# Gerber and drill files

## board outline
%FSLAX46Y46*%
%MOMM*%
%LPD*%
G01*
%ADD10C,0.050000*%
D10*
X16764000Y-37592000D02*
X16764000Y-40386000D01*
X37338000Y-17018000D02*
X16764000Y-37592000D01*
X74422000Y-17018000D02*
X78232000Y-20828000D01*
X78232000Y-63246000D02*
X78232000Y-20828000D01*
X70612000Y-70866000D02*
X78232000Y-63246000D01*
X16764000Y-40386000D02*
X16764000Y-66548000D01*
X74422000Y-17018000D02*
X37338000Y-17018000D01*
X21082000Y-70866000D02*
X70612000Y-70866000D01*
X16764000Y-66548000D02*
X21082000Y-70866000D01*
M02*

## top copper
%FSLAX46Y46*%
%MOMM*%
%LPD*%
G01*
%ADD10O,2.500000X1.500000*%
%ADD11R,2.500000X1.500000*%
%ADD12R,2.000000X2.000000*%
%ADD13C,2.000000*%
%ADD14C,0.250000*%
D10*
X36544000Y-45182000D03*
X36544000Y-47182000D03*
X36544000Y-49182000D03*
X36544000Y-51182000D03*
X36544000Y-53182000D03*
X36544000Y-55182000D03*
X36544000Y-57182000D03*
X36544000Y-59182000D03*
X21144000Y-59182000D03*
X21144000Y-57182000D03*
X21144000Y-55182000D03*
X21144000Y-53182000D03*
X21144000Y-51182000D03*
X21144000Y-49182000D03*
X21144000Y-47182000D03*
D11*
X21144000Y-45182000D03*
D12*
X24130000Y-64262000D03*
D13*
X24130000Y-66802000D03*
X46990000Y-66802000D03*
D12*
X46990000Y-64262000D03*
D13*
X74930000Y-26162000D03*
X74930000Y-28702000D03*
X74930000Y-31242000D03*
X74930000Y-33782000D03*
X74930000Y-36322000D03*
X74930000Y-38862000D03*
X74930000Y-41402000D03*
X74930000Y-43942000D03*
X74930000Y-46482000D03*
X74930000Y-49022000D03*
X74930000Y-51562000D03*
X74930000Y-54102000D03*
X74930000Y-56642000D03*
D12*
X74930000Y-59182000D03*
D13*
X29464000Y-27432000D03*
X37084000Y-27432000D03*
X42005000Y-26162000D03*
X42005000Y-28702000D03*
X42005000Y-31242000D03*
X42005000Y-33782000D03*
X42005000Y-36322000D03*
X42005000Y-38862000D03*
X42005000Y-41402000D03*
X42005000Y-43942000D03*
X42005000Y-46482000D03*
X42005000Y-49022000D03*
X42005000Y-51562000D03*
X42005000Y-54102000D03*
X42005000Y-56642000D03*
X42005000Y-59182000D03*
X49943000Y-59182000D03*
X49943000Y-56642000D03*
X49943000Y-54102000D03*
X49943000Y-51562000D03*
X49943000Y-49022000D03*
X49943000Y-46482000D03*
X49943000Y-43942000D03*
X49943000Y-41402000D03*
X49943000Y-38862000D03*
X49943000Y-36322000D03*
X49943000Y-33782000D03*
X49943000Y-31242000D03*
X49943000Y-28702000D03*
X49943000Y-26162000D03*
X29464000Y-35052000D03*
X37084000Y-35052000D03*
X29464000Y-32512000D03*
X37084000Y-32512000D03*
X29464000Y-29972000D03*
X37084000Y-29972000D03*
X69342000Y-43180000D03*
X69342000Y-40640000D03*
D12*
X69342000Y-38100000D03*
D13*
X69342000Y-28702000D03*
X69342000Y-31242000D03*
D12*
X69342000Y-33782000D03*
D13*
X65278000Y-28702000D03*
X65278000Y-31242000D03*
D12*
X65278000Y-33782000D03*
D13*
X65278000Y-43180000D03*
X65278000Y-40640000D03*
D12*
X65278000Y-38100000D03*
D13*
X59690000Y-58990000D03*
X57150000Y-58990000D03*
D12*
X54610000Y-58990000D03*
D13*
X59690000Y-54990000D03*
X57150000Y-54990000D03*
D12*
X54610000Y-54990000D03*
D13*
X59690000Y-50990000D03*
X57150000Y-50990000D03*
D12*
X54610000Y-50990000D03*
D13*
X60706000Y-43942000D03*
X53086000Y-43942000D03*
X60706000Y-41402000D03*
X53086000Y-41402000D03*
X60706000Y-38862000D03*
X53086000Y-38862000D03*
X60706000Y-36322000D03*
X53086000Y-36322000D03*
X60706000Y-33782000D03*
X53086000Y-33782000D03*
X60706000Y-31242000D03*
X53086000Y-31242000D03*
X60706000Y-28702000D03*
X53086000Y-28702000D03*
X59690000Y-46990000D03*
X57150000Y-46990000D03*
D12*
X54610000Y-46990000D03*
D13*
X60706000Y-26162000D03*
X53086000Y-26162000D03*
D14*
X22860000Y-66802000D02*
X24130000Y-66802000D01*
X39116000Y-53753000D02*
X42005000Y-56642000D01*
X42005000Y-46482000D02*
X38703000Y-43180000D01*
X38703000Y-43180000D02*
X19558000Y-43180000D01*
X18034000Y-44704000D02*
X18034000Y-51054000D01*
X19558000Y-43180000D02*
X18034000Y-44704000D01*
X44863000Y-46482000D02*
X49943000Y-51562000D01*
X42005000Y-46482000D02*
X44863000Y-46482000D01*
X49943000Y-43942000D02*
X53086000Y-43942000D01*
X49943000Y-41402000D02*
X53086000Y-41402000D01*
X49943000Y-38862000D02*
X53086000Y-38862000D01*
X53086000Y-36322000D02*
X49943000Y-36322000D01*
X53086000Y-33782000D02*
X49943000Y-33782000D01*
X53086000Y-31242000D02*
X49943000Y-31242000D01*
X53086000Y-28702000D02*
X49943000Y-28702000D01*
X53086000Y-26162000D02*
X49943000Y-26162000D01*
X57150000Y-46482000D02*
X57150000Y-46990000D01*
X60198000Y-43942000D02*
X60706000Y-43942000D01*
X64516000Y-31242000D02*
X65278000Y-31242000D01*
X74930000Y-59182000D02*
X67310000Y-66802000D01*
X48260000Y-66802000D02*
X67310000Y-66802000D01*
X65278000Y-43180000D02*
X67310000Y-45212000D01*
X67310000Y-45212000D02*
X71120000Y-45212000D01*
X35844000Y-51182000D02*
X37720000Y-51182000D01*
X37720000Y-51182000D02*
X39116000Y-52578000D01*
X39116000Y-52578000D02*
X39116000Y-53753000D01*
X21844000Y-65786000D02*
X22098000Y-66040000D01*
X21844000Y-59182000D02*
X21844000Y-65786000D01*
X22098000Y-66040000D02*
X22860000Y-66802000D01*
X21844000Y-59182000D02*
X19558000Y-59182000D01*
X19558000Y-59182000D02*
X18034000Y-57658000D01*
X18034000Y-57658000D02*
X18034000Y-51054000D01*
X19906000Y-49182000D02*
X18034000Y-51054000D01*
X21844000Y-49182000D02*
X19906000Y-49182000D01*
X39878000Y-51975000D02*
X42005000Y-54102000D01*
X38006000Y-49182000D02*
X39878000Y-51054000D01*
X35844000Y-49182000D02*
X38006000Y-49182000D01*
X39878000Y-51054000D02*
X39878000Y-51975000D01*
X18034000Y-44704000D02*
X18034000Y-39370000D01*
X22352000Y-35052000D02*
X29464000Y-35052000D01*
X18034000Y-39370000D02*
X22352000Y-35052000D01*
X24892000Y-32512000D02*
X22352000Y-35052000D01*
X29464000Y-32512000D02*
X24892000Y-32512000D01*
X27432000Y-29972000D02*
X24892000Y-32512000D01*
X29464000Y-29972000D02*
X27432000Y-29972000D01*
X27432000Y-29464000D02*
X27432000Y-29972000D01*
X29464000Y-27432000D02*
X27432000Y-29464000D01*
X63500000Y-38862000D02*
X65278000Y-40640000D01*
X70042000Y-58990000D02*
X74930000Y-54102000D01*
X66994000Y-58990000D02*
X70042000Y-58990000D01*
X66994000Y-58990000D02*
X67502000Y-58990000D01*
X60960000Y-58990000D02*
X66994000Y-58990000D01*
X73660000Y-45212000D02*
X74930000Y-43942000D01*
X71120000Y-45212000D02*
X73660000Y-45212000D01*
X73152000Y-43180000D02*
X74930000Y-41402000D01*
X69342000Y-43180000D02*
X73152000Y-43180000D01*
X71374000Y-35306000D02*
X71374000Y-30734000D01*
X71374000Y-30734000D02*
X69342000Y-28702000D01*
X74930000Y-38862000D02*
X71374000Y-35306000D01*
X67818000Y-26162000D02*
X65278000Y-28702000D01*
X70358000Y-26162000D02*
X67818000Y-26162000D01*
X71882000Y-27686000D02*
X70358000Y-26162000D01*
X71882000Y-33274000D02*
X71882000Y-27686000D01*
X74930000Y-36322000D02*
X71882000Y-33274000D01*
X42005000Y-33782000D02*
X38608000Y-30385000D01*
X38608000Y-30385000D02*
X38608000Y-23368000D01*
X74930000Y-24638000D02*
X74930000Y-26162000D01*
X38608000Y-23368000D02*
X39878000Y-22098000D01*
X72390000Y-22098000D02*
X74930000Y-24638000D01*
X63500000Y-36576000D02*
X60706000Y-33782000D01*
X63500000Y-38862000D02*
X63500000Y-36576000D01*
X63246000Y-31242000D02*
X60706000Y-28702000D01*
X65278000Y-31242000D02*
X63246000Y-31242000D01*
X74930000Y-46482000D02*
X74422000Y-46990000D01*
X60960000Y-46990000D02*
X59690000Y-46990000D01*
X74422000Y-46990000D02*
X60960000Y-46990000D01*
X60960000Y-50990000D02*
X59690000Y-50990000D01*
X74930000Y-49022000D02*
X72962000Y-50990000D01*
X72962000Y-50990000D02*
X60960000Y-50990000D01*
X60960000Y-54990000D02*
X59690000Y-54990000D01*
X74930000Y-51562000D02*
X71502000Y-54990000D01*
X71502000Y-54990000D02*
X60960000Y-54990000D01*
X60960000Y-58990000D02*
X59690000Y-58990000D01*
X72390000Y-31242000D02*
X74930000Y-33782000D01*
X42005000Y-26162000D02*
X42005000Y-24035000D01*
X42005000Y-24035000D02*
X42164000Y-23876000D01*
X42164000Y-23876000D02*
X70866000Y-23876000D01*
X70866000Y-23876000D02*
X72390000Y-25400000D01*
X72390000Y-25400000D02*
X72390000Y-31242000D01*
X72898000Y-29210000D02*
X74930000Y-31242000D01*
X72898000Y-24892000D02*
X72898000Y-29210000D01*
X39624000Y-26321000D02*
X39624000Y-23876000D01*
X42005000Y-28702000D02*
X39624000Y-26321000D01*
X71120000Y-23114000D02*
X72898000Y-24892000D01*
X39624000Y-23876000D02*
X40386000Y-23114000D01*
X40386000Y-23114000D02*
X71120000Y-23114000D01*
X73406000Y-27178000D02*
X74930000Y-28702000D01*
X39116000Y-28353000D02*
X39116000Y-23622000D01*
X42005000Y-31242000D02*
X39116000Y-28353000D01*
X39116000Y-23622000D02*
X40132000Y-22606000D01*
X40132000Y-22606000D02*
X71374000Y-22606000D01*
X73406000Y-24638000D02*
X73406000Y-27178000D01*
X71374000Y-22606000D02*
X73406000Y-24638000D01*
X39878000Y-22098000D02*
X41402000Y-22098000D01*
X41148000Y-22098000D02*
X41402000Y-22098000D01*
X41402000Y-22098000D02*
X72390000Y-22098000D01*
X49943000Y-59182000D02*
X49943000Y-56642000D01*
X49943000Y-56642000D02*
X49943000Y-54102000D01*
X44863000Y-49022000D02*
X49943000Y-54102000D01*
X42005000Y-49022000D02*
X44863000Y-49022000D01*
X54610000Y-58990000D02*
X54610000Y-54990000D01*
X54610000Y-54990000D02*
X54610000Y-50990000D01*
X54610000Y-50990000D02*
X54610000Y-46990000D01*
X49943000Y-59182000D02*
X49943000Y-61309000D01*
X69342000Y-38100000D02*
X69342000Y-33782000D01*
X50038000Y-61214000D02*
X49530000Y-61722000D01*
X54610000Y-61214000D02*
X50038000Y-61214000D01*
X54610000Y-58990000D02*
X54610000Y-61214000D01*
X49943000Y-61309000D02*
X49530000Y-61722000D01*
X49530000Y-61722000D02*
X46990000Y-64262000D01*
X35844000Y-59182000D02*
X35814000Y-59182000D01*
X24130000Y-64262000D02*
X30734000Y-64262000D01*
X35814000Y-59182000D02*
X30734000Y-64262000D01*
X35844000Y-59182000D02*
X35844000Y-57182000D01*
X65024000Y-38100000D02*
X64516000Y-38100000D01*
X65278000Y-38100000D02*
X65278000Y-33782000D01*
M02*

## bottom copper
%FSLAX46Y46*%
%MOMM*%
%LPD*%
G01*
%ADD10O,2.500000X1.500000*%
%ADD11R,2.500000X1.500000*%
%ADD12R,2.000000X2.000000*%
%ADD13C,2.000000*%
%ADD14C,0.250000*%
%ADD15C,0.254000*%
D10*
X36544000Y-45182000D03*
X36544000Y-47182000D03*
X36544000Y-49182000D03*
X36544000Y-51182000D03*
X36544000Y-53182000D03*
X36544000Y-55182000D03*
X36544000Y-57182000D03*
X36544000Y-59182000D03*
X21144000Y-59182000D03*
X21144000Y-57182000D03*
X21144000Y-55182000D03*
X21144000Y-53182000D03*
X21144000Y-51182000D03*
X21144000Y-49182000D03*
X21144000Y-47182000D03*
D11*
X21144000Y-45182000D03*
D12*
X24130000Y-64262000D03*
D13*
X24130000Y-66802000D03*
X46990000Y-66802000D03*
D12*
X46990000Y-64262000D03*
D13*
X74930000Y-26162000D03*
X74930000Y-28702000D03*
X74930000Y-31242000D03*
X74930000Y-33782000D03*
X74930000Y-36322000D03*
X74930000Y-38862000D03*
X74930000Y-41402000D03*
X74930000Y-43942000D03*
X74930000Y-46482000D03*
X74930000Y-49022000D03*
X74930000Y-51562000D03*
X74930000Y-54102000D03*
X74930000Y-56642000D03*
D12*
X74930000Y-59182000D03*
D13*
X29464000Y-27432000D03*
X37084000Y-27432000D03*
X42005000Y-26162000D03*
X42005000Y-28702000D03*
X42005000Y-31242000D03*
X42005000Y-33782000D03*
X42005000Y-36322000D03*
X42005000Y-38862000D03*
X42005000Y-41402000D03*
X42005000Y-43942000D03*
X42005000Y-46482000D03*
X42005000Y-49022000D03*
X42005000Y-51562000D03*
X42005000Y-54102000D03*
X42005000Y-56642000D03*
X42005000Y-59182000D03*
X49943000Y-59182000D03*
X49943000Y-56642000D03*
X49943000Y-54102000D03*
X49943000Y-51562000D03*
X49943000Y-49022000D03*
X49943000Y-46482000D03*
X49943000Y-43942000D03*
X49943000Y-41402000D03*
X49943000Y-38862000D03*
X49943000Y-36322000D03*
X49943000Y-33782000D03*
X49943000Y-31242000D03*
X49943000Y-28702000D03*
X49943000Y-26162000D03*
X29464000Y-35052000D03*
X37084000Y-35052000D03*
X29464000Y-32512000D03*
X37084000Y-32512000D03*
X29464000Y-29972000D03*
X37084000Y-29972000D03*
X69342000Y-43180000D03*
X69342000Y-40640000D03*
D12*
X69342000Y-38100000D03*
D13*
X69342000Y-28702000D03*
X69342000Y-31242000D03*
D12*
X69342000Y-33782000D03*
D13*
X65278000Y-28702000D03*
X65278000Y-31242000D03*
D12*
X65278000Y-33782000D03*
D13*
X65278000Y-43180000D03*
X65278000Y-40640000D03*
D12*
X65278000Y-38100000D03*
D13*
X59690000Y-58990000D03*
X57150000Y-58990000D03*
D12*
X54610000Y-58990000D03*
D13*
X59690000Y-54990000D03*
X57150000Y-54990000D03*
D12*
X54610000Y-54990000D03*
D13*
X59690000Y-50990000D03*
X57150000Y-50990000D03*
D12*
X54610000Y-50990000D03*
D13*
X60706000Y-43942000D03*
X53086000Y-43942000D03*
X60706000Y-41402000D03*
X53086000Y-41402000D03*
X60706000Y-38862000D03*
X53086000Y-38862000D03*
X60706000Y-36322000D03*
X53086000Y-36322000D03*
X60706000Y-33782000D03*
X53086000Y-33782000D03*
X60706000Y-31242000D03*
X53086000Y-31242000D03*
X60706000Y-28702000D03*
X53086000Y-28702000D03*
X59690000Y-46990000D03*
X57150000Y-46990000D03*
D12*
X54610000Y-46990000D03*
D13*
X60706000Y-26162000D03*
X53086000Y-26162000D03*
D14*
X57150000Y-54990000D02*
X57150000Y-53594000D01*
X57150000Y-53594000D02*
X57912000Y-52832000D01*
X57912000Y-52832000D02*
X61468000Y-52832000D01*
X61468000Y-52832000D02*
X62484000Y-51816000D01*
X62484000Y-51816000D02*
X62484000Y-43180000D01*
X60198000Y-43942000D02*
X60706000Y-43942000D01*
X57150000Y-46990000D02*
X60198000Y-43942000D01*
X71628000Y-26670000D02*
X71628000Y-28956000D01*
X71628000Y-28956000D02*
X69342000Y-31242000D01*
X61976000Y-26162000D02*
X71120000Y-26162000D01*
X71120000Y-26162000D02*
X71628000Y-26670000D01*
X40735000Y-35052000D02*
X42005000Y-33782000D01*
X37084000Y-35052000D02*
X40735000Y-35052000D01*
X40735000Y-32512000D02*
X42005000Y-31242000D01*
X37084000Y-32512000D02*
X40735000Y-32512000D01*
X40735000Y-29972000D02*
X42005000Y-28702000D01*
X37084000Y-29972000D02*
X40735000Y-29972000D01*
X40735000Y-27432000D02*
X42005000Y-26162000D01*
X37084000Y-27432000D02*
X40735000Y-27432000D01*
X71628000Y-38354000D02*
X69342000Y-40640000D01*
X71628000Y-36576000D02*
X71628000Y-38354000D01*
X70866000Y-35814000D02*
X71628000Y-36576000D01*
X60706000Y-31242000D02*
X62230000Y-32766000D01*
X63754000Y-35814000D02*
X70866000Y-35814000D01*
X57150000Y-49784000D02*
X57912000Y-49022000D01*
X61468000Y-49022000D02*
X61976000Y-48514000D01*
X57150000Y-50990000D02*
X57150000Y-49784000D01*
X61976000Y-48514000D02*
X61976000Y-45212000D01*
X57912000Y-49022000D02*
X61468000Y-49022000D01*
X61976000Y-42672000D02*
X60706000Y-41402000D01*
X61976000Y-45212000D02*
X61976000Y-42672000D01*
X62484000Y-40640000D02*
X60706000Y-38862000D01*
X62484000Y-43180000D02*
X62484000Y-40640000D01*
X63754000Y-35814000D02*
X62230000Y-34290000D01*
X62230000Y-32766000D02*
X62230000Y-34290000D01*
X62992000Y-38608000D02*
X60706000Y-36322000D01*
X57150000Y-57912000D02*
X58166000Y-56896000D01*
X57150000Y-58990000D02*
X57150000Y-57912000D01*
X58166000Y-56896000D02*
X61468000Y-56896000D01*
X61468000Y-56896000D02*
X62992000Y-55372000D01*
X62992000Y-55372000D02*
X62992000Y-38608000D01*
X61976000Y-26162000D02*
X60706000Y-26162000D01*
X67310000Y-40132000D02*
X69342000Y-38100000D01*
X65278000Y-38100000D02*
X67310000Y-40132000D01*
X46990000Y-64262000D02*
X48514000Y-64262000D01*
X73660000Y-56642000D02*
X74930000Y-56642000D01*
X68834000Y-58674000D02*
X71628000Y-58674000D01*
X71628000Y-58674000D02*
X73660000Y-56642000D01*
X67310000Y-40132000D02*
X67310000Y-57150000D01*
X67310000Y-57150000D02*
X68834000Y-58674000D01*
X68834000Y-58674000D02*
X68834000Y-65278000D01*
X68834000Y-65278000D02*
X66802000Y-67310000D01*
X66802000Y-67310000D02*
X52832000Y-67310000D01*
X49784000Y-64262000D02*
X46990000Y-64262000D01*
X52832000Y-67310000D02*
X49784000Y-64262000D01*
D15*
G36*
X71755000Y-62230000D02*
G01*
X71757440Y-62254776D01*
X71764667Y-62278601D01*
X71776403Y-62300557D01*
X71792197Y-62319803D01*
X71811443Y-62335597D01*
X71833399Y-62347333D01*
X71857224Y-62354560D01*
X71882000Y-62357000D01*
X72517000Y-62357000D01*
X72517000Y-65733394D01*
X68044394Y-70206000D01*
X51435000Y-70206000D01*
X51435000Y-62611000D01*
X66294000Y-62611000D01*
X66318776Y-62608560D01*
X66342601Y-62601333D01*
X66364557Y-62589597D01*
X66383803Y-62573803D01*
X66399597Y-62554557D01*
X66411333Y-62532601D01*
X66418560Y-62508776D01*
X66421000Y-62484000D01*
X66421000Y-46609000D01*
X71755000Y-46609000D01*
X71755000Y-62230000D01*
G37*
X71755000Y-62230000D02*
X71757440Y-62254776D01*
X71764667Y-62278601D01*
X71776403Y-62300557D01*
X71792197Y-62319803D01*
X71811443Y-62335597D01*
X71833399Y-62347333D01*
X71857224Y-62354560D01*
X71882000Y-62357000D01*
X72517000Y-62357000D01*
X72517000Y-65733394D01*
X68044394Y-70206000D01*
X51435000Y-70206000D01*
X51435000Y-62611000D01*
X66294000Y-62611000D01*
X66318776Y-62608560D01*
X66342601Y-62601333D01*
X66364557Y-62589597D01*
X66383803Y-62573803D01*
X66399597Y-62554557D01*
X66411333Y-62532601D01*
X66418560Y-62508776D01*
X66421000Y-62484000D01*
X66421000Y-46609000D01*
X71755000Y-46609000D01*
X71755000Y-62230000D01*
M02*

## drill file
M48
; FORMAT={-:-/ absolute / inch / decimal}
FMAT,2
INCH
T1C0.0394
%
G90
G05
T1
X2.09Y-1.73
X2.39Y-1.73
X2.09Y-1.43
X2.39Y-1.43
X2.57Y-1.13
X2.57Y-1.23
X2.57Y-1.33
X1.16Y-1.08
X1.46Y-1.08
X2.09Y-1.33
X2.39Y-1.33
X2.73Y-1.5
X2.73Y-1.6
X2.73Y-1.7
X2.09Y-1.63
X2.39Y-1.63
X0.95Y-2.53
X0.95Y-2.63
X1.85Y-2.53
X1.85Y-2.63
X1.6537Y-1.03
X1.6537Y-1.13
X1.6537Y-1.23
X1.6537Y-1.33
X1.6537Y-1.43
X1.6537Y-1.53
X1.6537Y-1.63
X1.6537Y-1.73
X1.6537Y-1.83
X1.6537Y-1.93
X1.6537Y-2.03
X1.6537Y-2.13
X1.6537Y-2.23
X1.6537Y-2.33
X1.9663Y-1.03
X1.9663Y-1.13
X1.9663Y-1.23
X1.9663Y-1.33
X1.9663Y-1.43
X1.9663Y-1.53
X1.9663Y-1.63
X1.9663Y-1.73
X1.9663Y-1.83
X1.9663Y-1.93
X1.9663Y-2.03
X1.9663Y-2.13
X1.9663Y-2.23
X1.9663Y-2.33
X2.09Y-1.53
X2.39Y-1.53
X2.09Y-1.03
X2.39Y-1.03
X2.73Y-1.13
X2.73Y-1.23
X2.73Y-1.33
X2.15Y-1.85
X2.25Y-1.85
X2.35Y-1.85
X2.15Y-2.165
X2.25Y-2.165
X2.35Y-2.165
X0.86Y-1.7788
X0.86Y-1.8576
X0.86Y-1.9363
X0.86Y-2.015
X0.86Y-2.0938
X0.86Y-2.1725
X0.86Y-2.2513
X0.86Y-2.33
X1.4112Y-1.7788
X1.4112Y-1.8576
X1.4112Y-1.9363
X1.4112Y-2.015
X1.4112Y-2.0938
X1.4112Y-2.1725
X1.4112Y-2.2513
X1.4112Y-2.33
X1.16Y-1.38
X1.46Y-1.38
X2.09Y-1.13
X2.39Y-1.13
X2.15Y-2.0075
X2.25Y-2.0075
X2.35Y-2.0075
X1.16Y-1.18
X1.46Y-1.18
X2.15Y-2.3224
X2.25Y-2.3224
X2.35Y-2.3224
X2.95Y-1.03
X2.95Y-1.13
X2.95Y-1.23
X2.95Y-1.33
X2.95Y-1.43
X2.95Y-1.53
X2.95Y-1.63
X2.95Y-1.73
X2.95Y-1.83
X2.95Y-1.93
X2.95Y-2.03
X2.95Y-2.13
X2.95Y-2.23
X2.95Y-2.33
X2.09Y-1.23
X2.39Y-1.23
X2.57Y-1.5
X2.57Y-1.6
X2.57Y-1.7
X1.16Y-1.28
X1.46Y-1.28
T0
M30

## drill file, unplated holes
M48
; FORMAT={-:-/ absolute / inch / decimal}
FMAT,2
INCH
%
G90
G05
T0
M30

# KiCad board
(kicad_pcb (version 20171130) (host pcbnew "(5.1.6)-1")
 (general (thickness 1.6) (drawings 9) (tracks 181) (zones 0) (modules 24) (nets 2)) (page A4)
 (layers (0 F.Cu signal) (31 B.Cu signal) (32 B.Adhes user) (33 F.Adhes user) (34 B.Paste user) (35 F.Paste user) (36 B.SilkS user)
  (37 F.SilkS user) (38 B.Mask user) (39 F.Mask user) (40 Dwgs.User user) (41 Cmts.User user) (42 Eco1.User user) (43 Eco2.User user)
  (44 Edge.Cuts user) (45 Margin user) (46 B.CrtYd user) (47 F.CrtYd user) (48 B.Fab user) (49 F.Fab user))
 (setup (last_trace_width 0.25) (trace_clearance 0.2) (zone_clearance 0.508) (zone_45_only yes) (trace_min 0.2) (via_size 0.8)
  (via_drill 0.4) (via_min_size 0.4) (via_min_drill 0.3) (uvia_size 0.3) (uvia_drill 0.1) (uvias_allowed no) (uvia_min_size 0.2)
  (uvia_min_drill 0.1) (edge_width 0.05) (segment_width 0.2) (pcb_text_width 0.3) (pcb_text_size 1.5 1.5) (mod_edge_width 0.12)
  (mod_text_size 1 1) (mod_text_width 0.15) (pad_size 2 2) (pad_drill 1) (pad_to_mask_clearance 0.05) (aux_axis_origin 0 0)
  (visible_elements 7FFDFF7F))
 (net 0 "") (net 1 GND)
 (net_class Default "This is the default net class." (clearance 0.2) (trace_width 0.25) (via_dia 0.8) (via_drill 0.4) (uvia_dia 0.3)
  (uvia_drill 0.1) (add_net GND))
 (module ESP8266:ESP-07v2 (layer F.Cu) (at 21.844 45.182)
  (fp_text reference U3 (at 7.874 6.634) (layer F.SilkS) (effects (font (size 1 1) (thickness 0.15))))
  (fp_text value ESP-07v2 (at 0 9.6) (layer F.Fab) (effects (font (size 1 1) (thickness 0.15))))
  (pad 16 thru_hole oval (at 14 0) (size 2.5 1.5) (drill 1 (offset 0.7 0)) (layers *.Cu *.Mask F.Paste F.SilkS))
  (pad 15 thru_hole oval (at 14 2) (size 2.5 1.5) (drill 1 (offset 0.7 0)) (layers *.Cu *.Mask F.Paste F.SilkS))
  (pad 14 thru_hole oval (at 14 4) (size 2.5 1.5) (drill 1 (offset 0.7 0)) (layers *.Cu *.Mask F.Paste F.SilkS))
  (pad 13 thru_hole oval (at 14 6) (size 2.5 1.5) (drill 1 (offset 0.7 0)) (layers *.Cu *.Mask F.Paste F.SilkS))
  (pad 12 thru_hole oval (at 14 8) (size 2.5 1.5) (drill 1 (offset 0.7 0)) (layers *.Cu *.Mask F.Paste F.SilkS))
  (pad 11 thru_hole oval (at 14 10) (size 2.5 1.5) (drill 1 (offset 0.7 0)) (layers *.Cu *.Mask F.Paste F.SilkS))
  (pad 10 thru_hole oval (at 14 12) (size 2.5 1.5) (drill 1 (offset 0.7 0)) (layers *.Cu *.Mask F.Paste F.SilkS) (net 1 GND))
  (pad 9 thru_hole oval (at 14 14) (size 2.5 1.5) (drill 1 (offset 0.7 0)) (layers *.Cu *.Mask F.Paste F.SilkS) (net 1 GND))
  (pad 8 thru_hole oval (at 0 14) (size 2.5 1.5) (drill 1 (offset -0.7 0)) (layers *.Cu *.Mask F.Paste F.SilkS))
  (pad 7 thru_hole oval (at 0 12) (size 2.5 1.5) (drill 1 (offset -0.7 0)) (layers *.Cu *.Mask F.Paste F.SilkS))
  (pad 6 thru_hole oval (at 0 10) (size 2.5 1.5) (drill 1 (offset -0.7 0)) (layers *.Cu *.Mask F.Paste F.SilkS))
  (pad 5 thru_hole oval (at 0 8) (size 2.5 1.5) (drill 1 (offset -0.7 0)) (layers *.Cu *.Mask F.Paste F.SilkS))
  (pad 4 thru_hole oval (at 0 6) (size 2.5 1.5) (drill 1 (offset -0.7 0)) (layers *.Cu *.Mask F.Paste F.SilkS))
  (pad 3 thru_hole oval (at 0 4) (size 2.5 1.5) (drill 1 (offset -0.7 0)) (layers *.Cu *.Mask F.Paste F.SilkS))
  (pad 2 thru_hole oval (at 0 2) (size 2.5 1.5) (drill 1 (offset -0.7 0)) (layers *.Cu *.Mask F.Paste F.SilkS))
  (pad 1 thru_hole rect (at 0 0) (size 2.5 1.5) (drill 1 (offset -0.7 0)) (layers *.Cu *.Mask F.Paste F.SilkS)))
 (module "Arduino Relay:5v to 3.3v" (layer F.Cu) (at 35.56 65.532 270)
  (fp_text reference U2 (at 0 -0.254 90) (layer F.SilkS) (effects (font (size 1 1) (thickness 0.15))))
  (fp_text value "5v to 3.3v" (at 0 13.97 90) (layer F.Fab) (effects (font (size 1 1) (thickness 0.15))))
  (pad 1 thru_hole rect (at -1.27 11.43 270) (size 2 2) (drill 1) (layers *.Cu *.Mask) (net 1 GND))
  (pad 3 thru_hole circle (at 1.27 11.43 270) (size 2 2) (drill 1) (layers *.Cu *.Mask))
  (pad 2 thru_hole circle (at 1.27 -11.43 270) (size 2 2) (drill 1) (layers *.Cu *.Mask))
  (pad 1 thru_hole rect (at -1.27 -11.43 270) (size 2 2) (drill 1) (layers *.Cu *.Mask) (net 1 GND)))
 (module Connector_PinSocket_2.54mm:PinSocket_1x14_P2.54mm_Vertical (layer F.Cu) (at 74.93 59.182 180)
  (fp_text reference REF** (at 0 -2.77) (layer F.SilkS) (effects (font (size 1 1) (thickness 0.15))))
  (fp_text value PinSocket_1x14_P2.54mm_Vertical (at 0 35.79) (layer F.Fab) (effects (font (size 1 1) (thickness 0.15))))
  (pad 14 thru_hole circle (at 0 33.02 180) (size 2 2) (drill 1) (layers *.Cu *.Mask))
  (pad 13 thru_hole circle (at 0 30.48 180) (size 2 2) (drill 1) (layers *.Cu *.Mask))
  (pad 12 thru_hole circle (at 0 27.94 180) (size 2 2) (drill 1) (layers *.Cu *.Mask))
  (pad 11 thru_hole circle (at 0 25.4 180) (size 2 2) (drill 1) (layers *.Cu *.Mask))
  (pad 10 thru_hole circle (at 0 22.86 180) (size 2 2) (drill 1) (layers *.Cu *.Mask))
  (pad 9 thru_hole circle (at 0 20.32 180) (size 2 2) (drill 1) (layers *.Cu *.Mask))
  (pad 8 thru_hole circle (at 0 17.78 180) (size 2 2) (drill 1) (layers *.Cu *.Mask))
  (pad 7 thru_hole circle (at 0 15.24 180) (size 2 2) (drill 1) (layers *.Cu *.Mask))
  (pad 6 thru_hole circle (at 0 12.7 180) (size 2 2) (drill 1) (layers *.Cu *.Mask))
  (pad 5 thru_hole circle (at 0 10.16 180) (size 2 2) (drill 1) (layers *.Cu *.Mask))
  (pad 4 thru_hole circle (at 0 7.62 180) (size 2 2) (drill 1) (layers *.Cu *.Mask))
  (pad 3 thru_hole circle (at 0 5.08 180) (size 2 2) (drill 1) (layers *.Cu *.Mask))
  (pad 2 thru_hole circle (at 0 2.54 180) (size 2 2) (drill 1) (layers *.Cu *.Mask) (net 1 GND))
  (pad 1 thru_hole rect (at 0 0 180) (size 2 2) (drill 1) (layers *.Cu *.Mask)))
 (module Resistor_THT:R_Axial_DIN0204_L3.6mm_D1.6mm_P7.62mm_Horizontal (layer F.Cu) (at 37.084 27.432 180)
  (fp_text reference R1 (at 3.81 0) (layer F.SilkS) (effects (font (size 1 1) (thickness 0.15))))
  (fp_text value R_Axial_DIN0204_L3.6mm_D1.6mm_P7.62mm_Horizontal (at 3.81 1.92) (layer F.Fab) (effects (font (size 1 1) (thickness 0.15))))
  (pad 2 thru_hole circle (at 7.62 0 180) (size 2 2) (drill 1) (layers *.Cu *.Mask))
  (pad 1 thru_hole circle (at 0 0 180) (size 2 2) (drill 1) (layers *.Cu *.Mask)))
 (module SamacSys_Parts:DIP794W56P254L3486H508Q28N (layer F.Cu) (at 45.974 42.672)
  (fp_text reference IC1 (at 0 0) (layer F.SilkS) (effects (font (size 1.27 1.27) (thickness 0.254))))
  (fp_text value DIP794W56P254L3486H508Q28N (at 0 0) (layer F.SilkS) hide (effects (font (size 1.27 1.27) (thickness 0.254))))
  (pad 1 thru_hole circle (at -3.969 -16.51) (size 2 2) (drill 1) (layers *.Cu *.Mask))
  (pad 2 thru_hole circle (at -3.969 -13.97) (size 2 2) (drill 1) (layers *.Cu *.Mask))
  (pad 3 thru_hole circle (at -3.969 -11.43) (size 2 2) (drill 1) (layers *.Cu *.Mask))
  (pad 4 thru_hole circle (at -3.969 -8.89) (size 2 2) (drill 1) (layers *.Cu *.Mask))
  (pad 5 thru_hole circle (at -3.969 -6.35) (size 2 2) (drill 1) (layers *.Cu *.Mask))
  (pad 6 thru_hole circle (at -3.969 -3.81) (size 2 2) (drill 1) (layers *.Cu *.Mask))
  (pad 7 thru_hole circle (at -3.969 -1.27) (size 2 2) (drill 1) (layers *.Cu *.Mask))
  (pad 8 thru_hole circle (at -3.969 1.27) (size 2 2) (drill 1) (layers *.Cu *.Mask))
  (pad 9 thru_hole circle (at -3.969 3.81) (size 2 2) (drill 1) (layers *.Cu *.Mask))
  (pad 10 thru_hole circle (at -3.969 6.35) (size 2 2) (drill 1) (layers *.Cu *.Mask) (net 1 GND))
  (pad 11 thru_hole circle (at -3.969 8.89) (size 2 2) (drill 1) (layers *.Cu *.Mask))
  (pad 12 thru_hole circle (at -3.969 11.43) (size 2 2) (drill 1) (layers *.Cu *.Mask))
  (pad 13 thru_hole circle (at -3.969 13.97) (size 2 2) (drill 1) (layers *.Cu *.Mask))
  (pad 14 thru_hole circle (at -3.969 16.51) (size 2 2) (drill 1) (layers *.Cu *.Mask))
  (pad 15 thru_hole circle (at 3.969 16.51) (size 2 2) (drill 1) (layers *.Cu *.Mask) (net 1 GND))
  (pad 16 thru_hole circle (at 3.969 13.97) (size 2 2) (drill 1) (layers *.Cu *.Mask) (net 1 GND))
  (pad 17 thru_hole circle (at 3.969 11.43) (size 2 2) (drill 1) (layers *.Cu *.Mask) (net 1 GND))
  (pad 18 thru_hole circle (at 3.969 8.89) (size 2 2) (drill 1) (layers *.Cu *.Mask))
  (pad 19 thru_hole circle (at 3.969 6.35) (size 2 2) (drill 1) (layers *.Cu *.Mask))
  (pad 20 thru_hole circle (at 3.969 3.81) (size 2 2) (drill 1) (layers *.Cu *.Mask))
  (pad 21 thru_hole circle (at 3.969 1.27) (size 2 2) (drill 1) (layers *.Cu *.Mask))
  (pad 22 thru_hole circle (at 3.969 -1.27) (size 2 2) (drill 1) (layers *.Cu *.Mask))
  (pad 23 thru_hole circle (at 3.969 -3.81) (size 2 2) (drill 1) (layers *.Cu *.Mask))
  (pad 24 thru_hole circle (at 3.969 -6.35) (size 2 2) (drill 1) (layers *.Cu *.Mask))
  (pad 25 thru_hole circle (at 3.969 -8.89) (size 2 2) (drill 1) (layers *.Cu *.Mask))
  (pad 26 thru_hole circle (at 3.969 -11.43) (size 2 2) (drill 1) (layers *.Cu *.Mask))
  (pad 27 thru_hole circle (at 3.969 -13.97) (size 2 2) (drill 1) (layers *.Cu *.Mask))
  (pad 28 thru_hole circle (at 3.969 -16.51) (size 2 2) (drill 1) (layers *.Cu *.Mask)))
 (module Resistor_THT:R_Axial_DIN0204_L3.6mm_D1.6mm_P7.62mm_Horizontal (layer F.Cu) (at 37.084 35.052 180)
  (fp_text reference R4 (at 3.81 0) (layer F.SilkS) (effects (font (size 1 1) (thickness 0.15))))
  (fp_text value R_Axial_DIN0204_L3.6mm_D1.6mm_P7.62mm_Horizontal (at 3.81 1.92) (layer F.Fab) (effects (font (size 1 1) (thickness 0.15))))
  (pad 2 thru_hole circle (at 7.62 0 180) (size 2 2) (drill 1) (layers *.Cu *.Mask))
  (pad 1 thru_hole circle (at 0 0 180) (size 2 2) (drill 1) (layers *.Cu *.Mask)))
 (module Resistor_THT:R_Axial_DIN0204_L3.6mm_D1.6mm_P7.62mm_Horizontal (layer F.Cu) (at 37.084 32.512 180)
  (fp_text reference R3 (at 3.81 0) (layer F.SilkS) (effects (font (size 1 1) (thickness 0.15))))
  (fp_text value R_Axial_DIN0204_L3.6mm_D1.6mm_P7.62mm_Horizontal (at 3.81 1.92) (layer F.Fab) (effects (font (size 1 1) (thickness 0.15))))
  (pad 2 thru_hole circle (at 7.62 0 180) (size 2 2) (drill 1) (layers *.Cu *.Mask))
  (pad 1 thru_hole circle (at 0 0 180) (size 2 2) (drill 1) (layers *.Cu *.Mask)))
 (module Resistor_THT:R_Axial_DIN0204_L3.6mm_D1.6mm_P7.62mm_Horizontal (layer F.Cu) (at 37.084 29.972 180)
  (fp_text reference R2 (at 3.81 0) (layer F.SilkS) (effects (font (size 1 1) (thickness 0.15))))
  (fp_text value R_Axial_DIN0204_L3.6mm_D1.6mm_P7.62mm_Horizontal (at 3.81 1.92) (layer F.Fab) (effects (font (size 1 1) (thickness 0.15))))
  (pad 2 thru_hole circle (at 7.62 0 180) (size 2 2) (drill 1) (layers *.Cu *.Mask))
  (pad 1 thru_hole circle (at 0 0 180) (size 2 2) (drill 1) (layers *.Cu *.Mask)))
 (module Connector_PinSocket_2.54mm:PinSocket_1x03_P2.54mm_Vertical (layer F.Cu) (at 69.342 38.1)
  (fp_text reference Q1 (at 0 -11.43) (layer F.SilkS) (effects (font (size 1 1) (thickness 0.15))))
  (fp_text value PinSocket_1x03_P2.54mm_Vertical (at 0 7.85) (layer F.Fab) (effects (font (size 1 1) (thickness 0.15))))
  (pad 3 thru_hole circle (at 0 5.08) (size 2 2) (drill 1) (layers *.Cu *.Mask))
  (pad 2 thru_hole circle (at 0 2.54) (size 2 2) (drill 1) (layers *.Cu *.Mask))
  (pad 1 thru_hole rect (at 0 0) (size 2 2) (drill 1) (layers *.Cu *.Mask) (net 1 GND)))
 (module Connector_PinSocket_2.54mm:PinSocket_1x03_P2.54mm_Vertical (layer F.Cu) (at 69.342 33.782 180)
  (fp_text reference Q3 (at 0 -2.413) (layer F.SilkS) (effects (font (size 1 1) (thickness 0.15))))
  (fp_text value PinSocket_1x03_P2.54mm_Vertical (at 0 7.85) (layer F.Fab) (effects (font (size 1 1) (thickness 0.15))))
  (pad 3 thru_hole circle (at 0 5.08 180) (size 2 2) (drill 1) (layers *.Cu *.Mask))
  (pad 2 thru_hole circle (at 0 2.54 180) (size 2 2) (drill 1) (layers *.Cu *.Mask))
  (pad 1 thru_hole rect (at 0 0 180) (size 2 2) (drill 1) (layers *.Cu *.Mask) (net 1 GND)))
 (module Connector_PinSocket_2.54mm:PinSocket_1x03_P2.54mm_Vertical (layer F.Cu) (at 65.278 33.782 180)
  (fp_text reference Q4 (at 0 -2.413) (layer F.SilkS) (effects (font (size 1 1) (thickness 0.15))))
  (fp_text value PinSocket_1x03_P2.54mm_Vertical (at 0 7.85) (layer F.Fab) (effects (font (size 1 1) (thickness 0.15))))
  (pad 3 thru_hole circle (at 0 5.08 180) (size 2 2) (drill 1) (layers *.Cu *.Mask))
  (pad 2 thru_hole circle (at 0 2.54 180) (size 2 2) (drill 1) (layers *.Cu *.Mask))
  (pad 1 thru_hole rect (at 0 0 180) (size 2 2) (drill 1) (layers *.Cu *.Mask) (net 1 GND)))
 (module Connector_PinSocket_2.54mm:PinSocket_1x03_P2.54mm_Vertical (layer F.Cu) (at 65.278 38.1)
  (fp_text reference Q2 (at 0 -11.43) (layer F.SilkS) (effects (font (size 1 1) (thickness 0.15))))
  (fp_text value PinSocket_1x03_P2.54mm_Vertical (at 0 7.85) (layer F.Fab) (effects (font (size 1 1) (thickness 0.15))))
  (pad 3 thru_hole circle (at 0 5.08) (size 2 2) (drill 1) (layers *.Cu *.Mask))
  (pad 2 thru_hole circle (at 0 2.54) (size 2 2) (drill 1) (layers *.Cu *.Mask))
  (pad 1 thru_hole rect (at 0 0) (size 2 2) (drill 1) (layers *.Cu *.Mask) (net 1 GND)))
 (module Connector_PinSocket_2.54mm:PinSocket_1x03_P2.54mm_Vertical (layer F.Cu) (at 54.61 58.99 90)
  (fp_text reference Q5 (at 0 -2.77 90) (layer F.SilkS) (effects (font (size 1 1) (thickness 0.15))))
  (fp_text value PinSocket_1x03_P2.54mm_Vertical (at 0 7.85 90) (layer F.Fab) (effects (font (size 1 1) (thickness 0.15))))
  (pad 3 thru_hole circle (at 0 5.08 90) (size 2 2) (drill 1) (layers *.Cu *.Mask))
  (pad 2 thru_hole circle (at 0 2.54 90) (size 2 2) (drill 1) (layers *.Cu *.Mask))
  (pad 1 thru_hole rect (at 0 0 90) (size 2 2) (drill 1) (layers *.Cu *.Mask) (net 1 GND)))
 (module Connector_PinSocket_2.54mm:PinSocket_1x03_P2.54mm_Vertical (layer F.Cu) (at 54.61 54.99 90)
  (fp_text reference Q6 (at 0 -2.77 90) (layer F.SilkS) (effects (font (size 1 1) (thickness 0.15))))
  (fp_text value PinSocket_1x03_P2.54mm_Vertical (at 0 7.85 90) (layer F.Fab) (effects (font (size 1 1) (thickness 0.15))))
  (pad 3 thru_hole circle (at 0 5.08 90) (size 2 2) (drill 1) (layers *.Cu *.Mask))
  (pad 2 thru_hole circle (at 0 2.54 90) (size 2 2) (drill 1) (layers *.Cu *.Mask))
  (pad 1 thru_hole rect (at 0 0 90) (size 2 2) (drill 1) (layers *.Cu *.Mask) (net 1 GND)))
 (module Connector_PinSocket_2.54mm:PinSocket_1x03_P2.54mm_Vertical (layer F.Cu) (at 54.61 50.99 90)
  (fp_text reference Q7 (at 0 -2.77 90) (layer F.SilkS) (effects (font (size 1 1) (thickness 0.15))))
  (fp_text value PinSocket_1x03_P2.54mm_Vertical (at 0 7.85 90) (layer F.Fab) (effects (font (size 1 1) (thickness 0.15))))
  (pad 3 thru_hole circle (at 0 5.08 90) (size 2 2) (drill 1) (layers *.Cu *.Mask))
  (pad 2 thru_hole circle (at 0 2.54 90) (size 2 2) (drill 1) (layers *.Cu *.Mask))
  (pad 1 thru_hole rect (at 0 0 90) (size 2 2) (drill 1) (layers *.Cu *.Mask) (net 1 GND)))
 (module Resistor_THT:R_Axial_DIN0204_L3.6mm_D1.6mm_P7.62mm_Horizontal (layer F.Cu) (at 53.086 43.942)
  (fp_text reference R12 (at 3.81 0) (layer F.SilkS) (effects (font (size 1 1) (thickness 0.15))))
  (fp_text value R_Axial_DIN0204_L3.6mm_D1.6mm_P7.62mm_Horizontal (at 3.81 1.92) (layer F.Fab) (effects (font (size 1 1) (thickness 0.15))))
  (pad 2 thru_hole circle (at 7.62 0) (size 2 2) (drill 1) (layers *.Cu *.Mask))
  (pad 1 thru_hole circle (at 0 0) (size 2 2) (drill 1) (layers *.Cu *.Mask)))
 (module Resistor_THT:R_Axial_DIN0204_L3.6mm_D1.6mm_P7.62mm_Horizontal (layer F.Cu) (at 53.086 41.402)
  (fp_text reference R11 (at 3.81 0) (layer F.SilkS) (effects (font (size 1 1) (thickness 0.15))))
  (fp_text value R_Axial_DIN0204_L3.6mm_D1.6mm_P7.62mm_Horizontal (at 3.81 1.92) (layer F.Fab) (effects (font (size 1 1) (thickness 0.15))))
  (pad 2 thru_hole circle (at 7.62 0) (size 2 2) (drill 1) (layers *.Cu *.Mask))
  (pad 1 thru_hole circle (at 0 0) (size 2 2) (drill 1) (layers *.Cu *.Mask)))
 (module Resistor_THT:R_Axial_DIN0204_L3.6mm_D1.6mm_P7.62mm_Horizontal (layer F.Cu) (at 53.086 38.862)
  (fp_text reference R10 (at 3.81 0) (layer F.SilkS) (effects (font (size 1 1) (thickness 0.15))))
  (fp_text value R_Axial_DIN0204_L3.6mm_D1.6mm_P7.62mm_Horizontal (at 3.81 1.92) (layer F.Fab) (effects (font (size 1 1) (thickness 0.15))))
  (pad 2 thru_hole circle (at 7.62 0) (size 2 2) (drill 1) (layers *.Cu *.Mask))
  (pad 1 thru_hole circle (at 0 0) (size 2 2) (drill 1) (layers *.Cu *.Mask)))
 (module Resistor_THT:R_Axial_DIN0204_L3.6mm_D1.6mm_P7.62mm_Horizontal (layer F.Cu) (at 53.086 36.322)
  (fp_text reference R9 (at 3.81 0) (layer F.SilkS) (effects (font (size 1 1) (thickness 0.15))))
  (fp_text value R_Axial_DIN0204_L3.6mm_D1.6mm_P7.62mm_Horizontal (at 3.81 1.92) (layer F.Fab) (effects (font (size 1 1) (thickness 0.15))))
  (pad 2 thru_hole circle (at 7.62 0) (size 2 2) (drill 1) (layers *.Cu *.Mask))
  (pad 1 thru_hole circle (at 0 0) (size 2 2) (drill 1) (layers *.Cu *.Mask)))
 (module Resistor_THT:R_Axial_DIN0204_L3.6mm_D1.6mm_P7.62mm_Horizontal (layer F.Cu) (at 53.086 33.782)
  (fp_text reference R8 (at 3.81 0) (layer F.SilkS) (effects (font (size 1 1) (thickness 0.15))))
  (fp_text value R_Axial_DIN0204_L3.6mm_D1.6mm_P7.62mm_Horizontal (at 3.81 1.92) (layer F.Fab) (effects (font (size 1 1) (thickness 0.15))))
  (pad 2 thru_hole circle (at 7.62 0) (size 2 2) (drill 1) (layers *.Cu *.Mask))
  (pad 1 thru_hole circle (at 0 0) (size 2 2) (drill 1) (layers *.Cu *.Mask)))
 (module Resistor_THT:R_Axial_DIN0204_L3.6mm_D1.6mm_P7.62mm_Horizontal (layer F.Cu) (at 53.086 31.242)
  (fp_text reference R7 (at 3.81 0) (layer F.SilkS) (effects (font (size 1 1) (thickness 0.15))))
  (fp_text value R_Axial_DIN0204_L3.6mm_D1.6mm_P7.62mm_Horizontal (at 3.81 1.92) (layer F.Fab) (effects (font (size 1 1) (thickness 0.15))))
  (pad 2 thru_hole circle (at 7.62 0) (size 2 2) (drill 1) (layers *.Cu *.Mask))
  (pad 1 thru_hole circle (at 0 0) (size 2 2) (drill 1) (layers *.Cu *.Mask)))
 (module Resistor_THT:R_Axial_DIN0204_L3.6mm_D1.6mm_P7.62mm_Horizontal (layer F.Cu) (at 53.086 28.702)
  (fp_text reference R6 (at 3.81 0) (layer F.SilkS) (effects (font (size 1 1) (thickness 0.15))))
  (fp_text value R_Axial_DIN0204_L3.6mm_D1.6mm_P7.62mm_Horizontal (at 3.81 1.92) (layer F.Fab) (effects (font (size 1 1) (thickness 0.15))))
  (pad 2 thru_hole circle (at 7.62 0) (size 2 2) (drill 1) (layers *.Cu *.Mask))
  (pad 1 thru_hole circle (at 0 0) (size 2 2) (drill 1) (layers *.Cu *.Mask)))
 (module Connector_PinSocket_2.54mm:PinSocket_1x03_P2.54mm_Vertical (layer F.Cu) (at 54.61 46.99 90)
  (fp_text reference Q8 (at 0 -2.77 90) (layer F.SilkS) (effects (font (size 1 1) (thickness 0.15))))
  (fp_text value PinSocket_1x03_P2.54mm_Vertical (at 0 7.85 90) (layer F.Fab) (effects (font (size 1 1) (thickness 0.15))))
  (pad 3 thru_hole circle (at 0 5.08 90) (size 2 2) (drill 1) (layers *.Cu *.Mask))
  (pad 2 thru_hole circle (at 0 2.54 90) (size 2 2) (drill 1) (layers *.Cu *.Mask))
  (pad 1 thru_hole rect (at 0 0 90) (size 2 2) (drill 1) (layers *.Cu *.Mask) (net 1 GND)))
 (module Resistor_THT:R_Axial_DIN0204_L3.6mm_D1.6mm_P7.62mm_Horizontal (layer F.Cu) (at 53.086 26.162)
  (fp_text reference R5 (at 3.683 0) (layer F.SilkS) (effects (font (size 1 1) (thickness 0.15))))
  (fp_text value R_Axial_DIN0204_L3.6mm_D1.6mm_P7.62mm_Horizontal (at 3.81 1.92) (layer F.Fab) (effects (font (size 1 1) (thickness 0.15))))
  (pad 2 thru_hole circle (at 7.62 0) (size 2 2) (drill 1) (layers *.Cu *.Mask))
  (pad 1 thru_hole circle (at 0 0) (size 2 2) (drill 1) (layers *.Cu *.Mask)))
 (gr_line (start 16.764 37.592) (end 16.764 40.386) (layer Edge.Cuts) (width 0.05))
 (gr_line (start 37.338 17.018) (end 16.764 37.592) (layer Edge.Cuts) (width 0.05))
 (gr_line (start 74.422 17.018) (end 78.232 20.828) (layer Edge.Cuts) (width 0.05))
 (gr_line (start 78.232 63.246) (end 78.232 20.828) (layer Edge.Cuts) (width 0.05))
 (gr_line (start 70.612 70.866) (end 78.232 63.246) (layer Edge.Cuts) (width 0.05))
 (gr_line (start 16.764 40.386) (end 16.764 66.548) (layer Edge.Cuts) (width 0.05))
 (gr_line (start 74.422 17.018) (end 37.338 17.018) (layer Edge.Cuts) (width 0.05))
 (gr_line (start 21.082 70.866) (end 70.612 70.866) (layer Edge.Cuts) (width 0.05))
 (gr_line (start 16.764 66.548) (end 21.082 70.866) (layer Edge.Cuts) (width 0.05))
 (segment (start 22.86 66.802) (end 24.13 66.802) (width 0.25) (layer F.Cu) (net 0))
 (segment (start 39.116 53.753) (end 42.005 56.642) (width 0.25) (layer F.Cu) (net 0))
 (segment (start 42.005 46.482) (end 38.703 43.18) (width 0.25) (layer F.Cu) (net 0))
 (segment (start 38.703 43.18) (end 19.558 43.18) (width 0.25) (layer F.Cu) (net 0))
 (segment (start 18.034 44.704) (end 18.034 51.054) (width 0.25) (layer F.Cu) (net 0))
 (segment (start 19.558 43.18) (end 18.034 44.704) (width 0.25) (layer F.Cu) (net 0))
 (segment (start 44.863 46.482) (end 49.943 51.562) (width 0.25) (layer F.Cu) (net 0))
 (segment (start 42.005 46.482) (end 44.863 46.482) (width 0.25) (layer F.Cu) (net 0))
 (segment (start 49.943 43.942) (end 53.086 43.942) (width 0.25) (layer F.Cu) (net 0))
 (segment (start 49.943 41.402) (end 53.086 41.402) (width 0.25) (layer F.Cu) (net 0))
 (segment (start 49.943 38.862) (end 53.086 38.862) (width 0.25) (layer F.Cu) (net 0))
 (segment (start 53.086 36.322) (end 49.943 36.322) (width 0.25) (layer F.Cu) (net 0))
 (segment (start 53.086 33.782) (end 49.943 33.782) (width 0.25) (layer F.Cu) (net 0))
 (segment (start 53.086 31.242) (end 49.943 31.242) (width 0.25) (layer F.Cu) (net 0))
 (segment (start 53.086 28.702) (end 49.943 28.702) (width 0.25) (layer F.Cu) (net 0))
 (segment (start 53.086 26.162) (end 49.943 26.162) (width 0.25) (layer F.Cu) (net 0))
 (segment (start 57.15 46.482) (end 57.15 46.99) (width 0.25) (layer F.Cu) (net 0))
 (segment (start 57.15 54.99) (end 57.15 53.594) (width 0.25) (layer B.Cu) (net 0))
 (segment (start 57.15 53.594) (end 57.912 52.832) (width 0.25) (layer B.Cu) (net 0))
 (segment (start 57.912 52.832) (end 61.468 52.832) (width 0.25) (layer B.Cu) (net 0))
 (segment (start 61.468 52.832) (end 62.484 51.816) (width 0.25) (layer B.Cu) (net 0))
 (segment (start 62.484 51.816) (end 62.484 43.18) (width 0.25) (layer B.Cu) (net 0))
 (segment (start 60.198 43.942) (end 60.706 43.942) (width 0.25) (layer F.Cu) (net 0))
 (segment (start 60.198 43.942) (end 60.706 43.942) (width 0.25) (layer B.Cu) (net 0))
 (segment (start 57.15 46.99) (end 60.198 43.942) (width 0.25) (layer B.Cu) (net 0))
 (segment (start 64.516 31.242) (end 65.278 31.242) (width 0.25) (layer F.Cu) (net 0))
 (segment (start 71.628 26.67) (end 71.628 28.956) (width 0.25) (layer B.Cu) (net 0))
 (segment (start 71.628 28.956) (end 69.342 31.242) (width 0.25) (layer B.Cu) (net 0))
 (segment (start 61.976 26.162) (end 71.12 26.162) (width 0.25) (layer B.Cu) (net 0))
 (segment (start 71.12 26.162) (end 71.628 26.67) (width 0.25) (layer B.Cu) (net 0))
 (segment (start 74.93 59.182) (end 67.31 66.802) (width 0.25) (layer F.Cu) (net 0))
 (segment (start 48.26 66.802) (end 67.31 66.802) (width 0.25) (layer F.Cu) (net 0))
 (segment (start 65.278 43.18) (end 67.31 45.212) (width 0.25) (layer F.Cu) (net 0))
 (segment (start 67.31 45.212) (end 71.12 45.212) (width 0.25) (layer F.Cu) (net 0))
 (segment (start 35.844 51.182) (end 37.72 51.182) (width 0.25) (layer F.Cu) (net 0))
 (segment (start 37.72 51.182) (end 39.116 52.578) (width 0.25) (layer F.Cu) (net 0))
 (segment (start 39.116 52.578) (end 39.116 53.753) (width 0.25) (layer F.Cu) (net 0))
 (segment (start 21.844 65.786) (end 22.098 66.04) (width 0.25) (layer F.Cu) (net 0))
 (segment (start 21.844 59.182) (end 21.844 65.786) (width 0.25) (layer F.Cu) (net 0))
 (segment (start 22.098 66.04) (end 22.86 66.802) (width 0.25) (layer F.Cu) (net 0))
 (segment (start 21.844 59.182) (end 19.558 59.182) (width 0.25) (layer F.Cu) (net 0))
 (segment (start 19.558 59.182) (end 18.034 57.658) (width 0.25) (layer F.Cu) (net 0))
 (segment (start 18.034 57.658) (end 18.034 51.054) (width 0.25) (layer F.Cu) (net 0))
 (segment (start 19.906 49.182) (end 18.034 51.054) (width 0.25) (layer F.Cu) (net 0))
 (segment (start 21.844 49.182) (end 19.906 49.182) (width 0.25) (layer F.Cu) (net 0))
 (segment (start 39.878 51.975) (end 42.005 54.102) (width 0.25) (layer F.Cu) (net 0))
 (segment (start 38.006 49.182) (end 39.878 51.054) (width 0.25) (layer F.Cu) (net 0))
 (segment (start 35.844 49.182) (end 38.006 49.182) (width 0.25) (layer F.Cu) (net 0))
 (segment (start 39.878 51.054) (end 39.878 51.975) (width 0.25) (layer F.Cu) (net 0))
 (segment (start 18.034 44.704) (end 18.034 39.37) (width 0.25) (layer F.Cu) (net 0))
 (segment (start 22.352 35.052) (end 29.464 35.052) (width 0.25) (layer F.Cu) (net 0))
 (segment (start 18.034 39.37) (end 22.352 35.052) (width 0.25) (layer F.Cu) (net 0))
 (segment (start 24.892 32.512) (end 22.352 35.052) (width 0.25) (layer F.Cu) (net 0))
 (segment (start 29.464 32.512) (end 24.892 32.512) (width 0.25) (layer F.Cu) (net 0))
 (segment (start 27.432 29.972) (end 24.892 32.512) (width 0.25) (layer F.Cu) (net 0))
 (segment (start 29.464 29.972) (end 27.432 29.972) (width 0.25) (layer F.Cu) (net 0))
 (segment (start 27.432 29.464) (end 27.432 29.972) (width 0.25) (layer F.Cu) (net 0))
 (segment (start 29.464 27.432) (end 27.432 29.464) (width 0.25) (layer F.Cu) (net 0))
 (segment (start 40.735 35.052) (end 42.005 33.782) (width 0.25) (layer B.Cu) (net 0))
 (segment (start 37.084 35.052) (end 40.735 35.052) (width 0.25) (layer B.Cu) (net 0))
 (segment (start 40.735 32.512) (end 42.005 31.242) (width 0.25) (layer B.Cu) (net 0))
 (segment (start 37.084 32.512) (end 40.735 32.512) (width 0.25) (layer B.Cu) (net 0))
 (segment (start 40.735 29.972) (end 42.005 28.702) (width 0.25) (layer B.Cu) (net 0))
 (segment (start 37.084 29.972) (end 40.735 29.972) (width 0.25) (layer B.Cu) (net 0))
 (segment (start 40.735 27.432) (end 42.005 26.162) (width 0.25) (layer B.Cu) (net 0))
 (segment (start 37.084 27.432) (end 40.735 27.432) (width 0.25) (layer B.Cu) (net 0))
 (segment (start 63.5 38.862) (end 65.278 40.64) (width 0.25) (layer F.Cu) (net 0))
 (segment (start 71.628 38.354) (end 69.342 40.64) (width 0.25) (layer B.Cu) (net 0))
 (segment (start 71.628 36.576) (end 71.628 38.354) (width 0.25) (layer B.Cu) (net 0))
 (segment (start 70.866 35.814) (end 71.628 36.576) (width 0.25) (layer B.Cu) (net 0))
 (segment (start 60.706 31.242) (end 62.23 32.766) (width 0.25) (layer B.Cu) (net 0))
 (segment (start 63.754 35.814) (end 70.866 35.814) (width 0.25) (layer B.Cu) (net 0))
 (segment (start 70.042 58.99) (end 74.93 54.102) (width 0.25) (layer F.Cu) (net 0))
 (segment (start 66.994 58.99) (end 70.042 58.99) (width 0.25) (layer F.Cu) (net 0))
 (segment (start 66.994 58.99) (end 67.502 58.99) (width 0.25) (layer F.Cu) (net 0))
 (segment (start 60.96 58.99) (end 66.994 58.99) (width 0.25) (layer F.Cu) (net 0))
 (segment (start 73.66 45.212) (end 74.93 43.942) (width 0.25) (layer F.Cu) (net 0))
 (segment (start 71.12 45.212) (end 73.66 45.212) (width 0.25) (layer F.Cu) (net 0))
 (segment (start 73.152 43.18) (end 74.93 41.402) (width 0.25) (layer F.Cu) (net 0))
 (segment (start 69.342 43.18) (end 73.152 43.18) (width 0.25) (layer F.Cu) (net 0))
 (segment (start 71.374 35.306) (end 71.374 30.734) (width 0.25) (layer F.Cu) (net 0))
 (segment (start 71.374 30.734) (end 69.342 28.702) (width 0.25) (layer F.Cu) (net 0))
 (segment (start 74.93 38.862) (end 71.374 35.306) (width 0.25) (layer F.Cu) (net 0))
 (segment (start 67.818 26.162) (end 65.278 28.702) (width 0.25) (layer F.Cu) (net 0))
 (segment (start 70.358 26.162) (end 67.818 26.162) (width 0.25) (layer F.Cu) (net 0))
 (segment (start 71.882 27.686) (end 70.358 26.162) (width 0.25) (layer F.Cu) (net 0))
 (segment (start 71.882 33.274) (end 71.882 27.686) (width 0.25) (layer F.Cu) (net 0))
 (segment (start 74.93 36.322) (end 71.882 33.274) (width 0.25) (layer F.Cu) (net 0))
 (segment (start 42.005 33.782) (end 38.608 30.385) (width 0.25) (layer F.Cu) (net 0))
 (segment (start 38.608 30.385) (end 38.608 23.368) (width 0.25) (layer F.Cu) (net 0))
 (segment (start 74.93 24.638) (end 74.93 26.162) (width 0.25) (layer F.Cu) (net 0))
 (segment (start 38.608 23.368) (end 39.878 22.098) (width 0.25) (layer F.Cu) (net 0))
 (segment (start 72.39 22.098) (end 74.93 24.638) (width 0.25) (layer F.Cu) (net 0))
 (segment (start 57.15 49.784) (end 57.912 49.022) (width 0.25) (layer B.Cu) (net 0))
 (segment (start 61.468 49.022) (end 61.976 48.514) (width 0.25) (layer B.Cu) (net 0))
 (segment (start 57.15 50.99) (end 57.15 49.784) (width 0.25) (layer B.Cu) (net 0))
 (segment (start 61.976 48.514) (end 61.976 45.212) (width 0.25) (layer B.Cu) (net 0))
 (segment (start 57.912 49.022) (end 61.468 49.022) (width 0.25) (layer B.Cu) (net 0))
 (segment (start 61.976 42.672) (end 60.706 41.402) (width 0.25) (layer B.Cu) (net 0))
 (segment (start 61.976 45.212) (end 61.976 42.672) (width 0.25) (layer B.Cu) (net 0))
 (segment (start 62.484 40.64) (end 60.706 38.862) (width 0.25) (layer B.Cu) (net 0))
 (segment (start 62.484 43.18) (end 62.484 40.64) (width 0.25) (layer B.Cu) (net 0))
 (segment (start 63.754 35.814) (end 62.23 34.29) (width 0.25) (layer B.Cu) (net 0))
 (segment (start 62.23 32.766) (end 62.23 34.29) (width 0.25) (layer B.Cu) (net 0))
 (segment (start 62.992 38.608) (end 60.706 36.322) (width 0.25) (layer B.Cu) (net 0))
 (segment (start 57.15 57.912) (end 58.166 56.896) (width 0.25) (layer B.Cu) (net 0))
 (segment (start 57.15 58.99) (end 57.15 57.912) (width 0.25) (layer B.Cu) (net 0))
 (segment (start 58.166 56.896) (end 61.468 56.896) (width 0.25) (layer B.Cu) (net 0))
 (segment (start 61.468 56.896) (end 62.992 55.372) (width 0.25) (layer B.Cu) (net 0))
 (segment (start 62.992 55.372) (end 62.992 38.608) (width 0.25) (layer B.Cu) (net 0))
 (segment (start 63.5 36.576) (end 60.706 33.782) (width 0.25) (layer F.Cu) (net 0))
 (segment (start 63.5 38.862) (end 63.5 36.576) (width 0.25) (layer F.Cu) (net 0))
 (segment (start 63.246 31.242) (end 60.706 28.702) (width 0.25) (layer F.Cu) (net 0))
 (segment (start 65.278 31.242) (end 63.246 31.242) (width 0.25) (layer F.Cu) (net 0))
 (segment (start 61.976 26.162) (end 60.706 26.162) (width 0.25) (layer B.Cu) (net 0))
 (segment (start 74.93 46.482) (end 74.422 46.99) (width 0.25) (layer F.Cu) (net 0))
 (segment (start 60.96 46.99) (end 59.69 46.99) (width 0.25) (layer F.Cu) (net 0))
 (segment (start 74.422 46.99) (end 60.96 46.99) (width 0.25) (layer F.Cu) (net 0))
 (segment (start 60.96 50.99) (end 59.69 50.99) (width 0.25) (layer F.Cu) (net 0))
 (segment (start 74.93 49.022) (end 72.962 50.99) (width 0.25) (layer F.Cu) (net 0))
 (segment (start 72.962 50.99) (end 60.96 50.99) (width 0.25) (layer F.Cu) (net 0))
 (segment (start 60.96 54.99) (end 59.69 54.99) (width 0.25) (layer F.Cu) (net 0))
 (segment (start 74.93 51.562) (end 71.502 54.99) (width 0.25) (layer F.Cu) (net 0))
 (segment (start 71.502 54.99) (end 60.96 54.99) (width 0.25) (layer F.Cu) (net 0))
 (segment (start 60.96 58.99) (end 59.69 58.99) (width 0.25) (layer F.Cu) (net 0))
 (segment (start 72.39 31.242) (end 74.93 33.782) (width 0.25) (layer F.Cu) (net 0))
 (segment (start 42.005 26.162) (end 42.005 24.035) (width 0.25) (layer F.Cu) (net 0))
 (segment (start 42.005 24.035) (end 42.164 23.876) (width 0.25) (layer F.Cu) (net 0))
 (segment (start 42.164 23.876) (end 70.866 23.876) (width 0.25) (layer F.Cu) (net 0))
 (segment (start 70.866 23.876) (end 72.39 25.4) (width 0.25) (layer F.Cu) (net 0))
 (segment (start 72.39 25.4) (end 72.39 31.242) (width 0.25) (layer F.Cu) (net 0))
 (segment (start 72.898 29.21) (end 74.93 31.242) (width 0.25) (layer F.Cu) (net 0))
 (segment (start 72.898 24.892) (end 72.898 29.21) (width 0.25) (layer F.Cu) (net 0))
 (segment (start 39.624 26.321) (end 39.624 23.876) (width 0.25) (layer F.Cu) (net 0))
 (segment (start 42.005 28.702) (end 39.624 26.321) (width 0.25) (layer F.Cu) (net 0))
 (segment (start 71.12 23.114) (end 72.898 24.892) (width 0.25) (layer F.Cu) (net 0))
 (segment (start 39.624 23.876) (end 40.386 23.114) (width 0.25) (layer F.Cu) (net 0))
 (segment (start 40.386 23.114) (end 71.12 23.114) (width 0.25) (layer F.Cu) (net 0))
 (segment (start 73.406 27.178) (end 74.93 28.702) (width 0.25) (layer F.Cu) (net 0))
 (segment (start 39.116 28.353) (end 39.116 23.622) (width 0.25) (layer F.Cu) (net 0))
 (segment (start 42.005 31.242) (end 39.116 28.353) (width 0.25) (layer F.Cu) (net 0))
 (segment (start 39.116 23.622) (end 40.132 22.606) (width 0.25) (layer F.Cu) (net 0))
 (segment (start 40.132 22.606) (end 71.374 22.606) (width 0.25) (layer F.Cu) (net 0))
 (segment (start 73.406 24.638) (end 73.406 27.178) (width 0.25) (layer F.Cu) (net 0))
 (segment (start 71.374 22.606) (end 73.406 24.638) (width 0.25) (layer F.Cu) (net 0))
 (segment (start 39.878 22.098) (end 41.402 22.098) (width 0.25) (layer F.Cu) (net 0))
 (segment (start 41.148 22.098) (end 41.402 22.098) (width 0.25) (layer F.Cu) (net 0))
 (segment (start 41.402 22.098) (end 72.39 22.098) (width 0.25) (layer F.Cu) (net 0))
 (segment (start 49.943 59.182) (end 49.943 56.642) (width 0.25) (layer F.Cu) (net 1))
 (segment (start 49.943 56.642) (end 49.943 54.102) (width 0.25) (layer F.Cu) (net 1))
 (segment (start 44.863 49.022) (end 49.943 54.102) (width 0.25) (layer F.Cu) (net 1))
 (segment (start 42.005 49.022) (end 44.863 49.022) (width 0.25) (layer F.Cu) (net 1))
 (segment (start 54.61 58.99) (end 54.61 54.99) (width 0.25) (layer F.Cu) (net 1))
 (segment (start 54.61 54.99) (end 54.61 50.99) (width 0.25) (layer F.Cu) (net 1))
 (segment (start 54.61 50.99) (end 54.61 46.99) (width 0.25) (layer F.Cu) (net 1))
 (segment (start 49.943 59.182) (end 49.943 61.309) (width 0.25) (layer F.Cu) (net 1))
 (segment (start 69.342 38.1) (end 69.342 33.782) (width 0.25) (layer F.Cu) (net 1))
 (segment (start 50.038 61.214) (end 49.53 61.722) (width 0.25) (layer F.Cu) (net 1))
 (segment (start 54.61 61.214) (end 50.038 61.214) (width 0.25) (layer F.Cu) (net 1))
 (segment (start 54.61 58.99) (end 54.61 61.214) (width 0.25) (layer F.Cu) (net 1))
 (segment (start 49.943 61.309) (end 49.53 61.722) (width 0.25) (layer F.Cu) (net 1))
 (segment (start 49.53 61.722) (end 46.99 64.262) (width 0.25) (layer F.Cu) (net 1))
 (segment (start 67.31 40.132) (end 69.342 38.1) (width 0.25) (layer B.Cu) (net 1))
 (segment (start 65.278 38.1) (end 67.31 40.132) (width 0.25) (layer B.Cu) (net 1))
 (segment (start 35.844 59.182) (end 35.814 59.182) (width 0.25) (layer F.Cu) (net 1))
 (segment (start 24.13 64.262) (end 30.734 64.262) (width 0.25) (layer F.Cu) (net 1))
 (segment (start 35.814 59.182) (end 30.734 64.262) (width 0.25) (layer F.Cu) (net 1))
 (segment (start 35.844 59.182) (end 35.844 57.182) (width 0.25) (layer F.Cu) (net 1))
 (segment (start 46.99 64.262) (end 48.514 64.262) (width 0.25) (layer B.Cu) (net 1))
 (segment (start 65.024 38.1) (end 64.516 38.1) (width 0.25) (layer F.Cu) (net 1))
 (segment (start 65.278 38.1) (end 65.278 33.782) (width 0.25) (layer F.Cu) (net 1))
 (segment (start 73.66 56.642) (end 74.93 56.642) (width 0.25) (layer B.Cu) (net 1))
 (segment (start 68.834 58.674) (end 71.628 58.674) (width 0.25) (layer B.Cu) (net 1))
 (segment (start 71.628 58.674) (end 73.66 56.642) (width 0.25) (layer B.Cu) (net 1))
 (segment (start 67.31 40.132) (end 67.31 57.15) (width 0.25) (layer B.Cu) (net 1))
 (segment (start 67.31 57.15) (end 68.834 58.674) (width 0.25) (layer B.Cu) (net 1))
 (segment (start 68.834 58.674) (end 68.834 65.278) (width 0.25) (layer B.Cu) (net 1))
 (segment (start 68.834 65.278) (end 66.802 67.31) (width 0.25) (layer B.Cu) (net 1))
 (segment (start 66.802 67.31) (end 52.832 67.31) (width 0.25) (layer B.Cu) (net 1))
 (segment (start 49.784 64.262) (end 46.99 64.262) (width 0.25) (layer B.Cu) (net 1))
 (segment (start 52.832 67.31) (end 49.784 64.262) (width 0.25) (layer B.Cu) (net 1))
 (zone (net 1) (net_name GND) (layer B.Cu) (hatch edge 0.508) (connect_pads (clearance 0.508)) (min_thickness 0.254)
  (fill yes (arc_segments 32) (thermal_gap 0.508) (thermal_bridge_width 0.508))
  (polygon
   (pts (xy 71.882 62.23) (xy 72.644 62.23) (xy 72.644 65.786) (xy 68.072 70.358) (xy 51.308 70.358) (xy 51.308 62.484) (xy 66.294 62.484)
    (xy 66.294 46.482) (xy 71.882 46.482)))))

